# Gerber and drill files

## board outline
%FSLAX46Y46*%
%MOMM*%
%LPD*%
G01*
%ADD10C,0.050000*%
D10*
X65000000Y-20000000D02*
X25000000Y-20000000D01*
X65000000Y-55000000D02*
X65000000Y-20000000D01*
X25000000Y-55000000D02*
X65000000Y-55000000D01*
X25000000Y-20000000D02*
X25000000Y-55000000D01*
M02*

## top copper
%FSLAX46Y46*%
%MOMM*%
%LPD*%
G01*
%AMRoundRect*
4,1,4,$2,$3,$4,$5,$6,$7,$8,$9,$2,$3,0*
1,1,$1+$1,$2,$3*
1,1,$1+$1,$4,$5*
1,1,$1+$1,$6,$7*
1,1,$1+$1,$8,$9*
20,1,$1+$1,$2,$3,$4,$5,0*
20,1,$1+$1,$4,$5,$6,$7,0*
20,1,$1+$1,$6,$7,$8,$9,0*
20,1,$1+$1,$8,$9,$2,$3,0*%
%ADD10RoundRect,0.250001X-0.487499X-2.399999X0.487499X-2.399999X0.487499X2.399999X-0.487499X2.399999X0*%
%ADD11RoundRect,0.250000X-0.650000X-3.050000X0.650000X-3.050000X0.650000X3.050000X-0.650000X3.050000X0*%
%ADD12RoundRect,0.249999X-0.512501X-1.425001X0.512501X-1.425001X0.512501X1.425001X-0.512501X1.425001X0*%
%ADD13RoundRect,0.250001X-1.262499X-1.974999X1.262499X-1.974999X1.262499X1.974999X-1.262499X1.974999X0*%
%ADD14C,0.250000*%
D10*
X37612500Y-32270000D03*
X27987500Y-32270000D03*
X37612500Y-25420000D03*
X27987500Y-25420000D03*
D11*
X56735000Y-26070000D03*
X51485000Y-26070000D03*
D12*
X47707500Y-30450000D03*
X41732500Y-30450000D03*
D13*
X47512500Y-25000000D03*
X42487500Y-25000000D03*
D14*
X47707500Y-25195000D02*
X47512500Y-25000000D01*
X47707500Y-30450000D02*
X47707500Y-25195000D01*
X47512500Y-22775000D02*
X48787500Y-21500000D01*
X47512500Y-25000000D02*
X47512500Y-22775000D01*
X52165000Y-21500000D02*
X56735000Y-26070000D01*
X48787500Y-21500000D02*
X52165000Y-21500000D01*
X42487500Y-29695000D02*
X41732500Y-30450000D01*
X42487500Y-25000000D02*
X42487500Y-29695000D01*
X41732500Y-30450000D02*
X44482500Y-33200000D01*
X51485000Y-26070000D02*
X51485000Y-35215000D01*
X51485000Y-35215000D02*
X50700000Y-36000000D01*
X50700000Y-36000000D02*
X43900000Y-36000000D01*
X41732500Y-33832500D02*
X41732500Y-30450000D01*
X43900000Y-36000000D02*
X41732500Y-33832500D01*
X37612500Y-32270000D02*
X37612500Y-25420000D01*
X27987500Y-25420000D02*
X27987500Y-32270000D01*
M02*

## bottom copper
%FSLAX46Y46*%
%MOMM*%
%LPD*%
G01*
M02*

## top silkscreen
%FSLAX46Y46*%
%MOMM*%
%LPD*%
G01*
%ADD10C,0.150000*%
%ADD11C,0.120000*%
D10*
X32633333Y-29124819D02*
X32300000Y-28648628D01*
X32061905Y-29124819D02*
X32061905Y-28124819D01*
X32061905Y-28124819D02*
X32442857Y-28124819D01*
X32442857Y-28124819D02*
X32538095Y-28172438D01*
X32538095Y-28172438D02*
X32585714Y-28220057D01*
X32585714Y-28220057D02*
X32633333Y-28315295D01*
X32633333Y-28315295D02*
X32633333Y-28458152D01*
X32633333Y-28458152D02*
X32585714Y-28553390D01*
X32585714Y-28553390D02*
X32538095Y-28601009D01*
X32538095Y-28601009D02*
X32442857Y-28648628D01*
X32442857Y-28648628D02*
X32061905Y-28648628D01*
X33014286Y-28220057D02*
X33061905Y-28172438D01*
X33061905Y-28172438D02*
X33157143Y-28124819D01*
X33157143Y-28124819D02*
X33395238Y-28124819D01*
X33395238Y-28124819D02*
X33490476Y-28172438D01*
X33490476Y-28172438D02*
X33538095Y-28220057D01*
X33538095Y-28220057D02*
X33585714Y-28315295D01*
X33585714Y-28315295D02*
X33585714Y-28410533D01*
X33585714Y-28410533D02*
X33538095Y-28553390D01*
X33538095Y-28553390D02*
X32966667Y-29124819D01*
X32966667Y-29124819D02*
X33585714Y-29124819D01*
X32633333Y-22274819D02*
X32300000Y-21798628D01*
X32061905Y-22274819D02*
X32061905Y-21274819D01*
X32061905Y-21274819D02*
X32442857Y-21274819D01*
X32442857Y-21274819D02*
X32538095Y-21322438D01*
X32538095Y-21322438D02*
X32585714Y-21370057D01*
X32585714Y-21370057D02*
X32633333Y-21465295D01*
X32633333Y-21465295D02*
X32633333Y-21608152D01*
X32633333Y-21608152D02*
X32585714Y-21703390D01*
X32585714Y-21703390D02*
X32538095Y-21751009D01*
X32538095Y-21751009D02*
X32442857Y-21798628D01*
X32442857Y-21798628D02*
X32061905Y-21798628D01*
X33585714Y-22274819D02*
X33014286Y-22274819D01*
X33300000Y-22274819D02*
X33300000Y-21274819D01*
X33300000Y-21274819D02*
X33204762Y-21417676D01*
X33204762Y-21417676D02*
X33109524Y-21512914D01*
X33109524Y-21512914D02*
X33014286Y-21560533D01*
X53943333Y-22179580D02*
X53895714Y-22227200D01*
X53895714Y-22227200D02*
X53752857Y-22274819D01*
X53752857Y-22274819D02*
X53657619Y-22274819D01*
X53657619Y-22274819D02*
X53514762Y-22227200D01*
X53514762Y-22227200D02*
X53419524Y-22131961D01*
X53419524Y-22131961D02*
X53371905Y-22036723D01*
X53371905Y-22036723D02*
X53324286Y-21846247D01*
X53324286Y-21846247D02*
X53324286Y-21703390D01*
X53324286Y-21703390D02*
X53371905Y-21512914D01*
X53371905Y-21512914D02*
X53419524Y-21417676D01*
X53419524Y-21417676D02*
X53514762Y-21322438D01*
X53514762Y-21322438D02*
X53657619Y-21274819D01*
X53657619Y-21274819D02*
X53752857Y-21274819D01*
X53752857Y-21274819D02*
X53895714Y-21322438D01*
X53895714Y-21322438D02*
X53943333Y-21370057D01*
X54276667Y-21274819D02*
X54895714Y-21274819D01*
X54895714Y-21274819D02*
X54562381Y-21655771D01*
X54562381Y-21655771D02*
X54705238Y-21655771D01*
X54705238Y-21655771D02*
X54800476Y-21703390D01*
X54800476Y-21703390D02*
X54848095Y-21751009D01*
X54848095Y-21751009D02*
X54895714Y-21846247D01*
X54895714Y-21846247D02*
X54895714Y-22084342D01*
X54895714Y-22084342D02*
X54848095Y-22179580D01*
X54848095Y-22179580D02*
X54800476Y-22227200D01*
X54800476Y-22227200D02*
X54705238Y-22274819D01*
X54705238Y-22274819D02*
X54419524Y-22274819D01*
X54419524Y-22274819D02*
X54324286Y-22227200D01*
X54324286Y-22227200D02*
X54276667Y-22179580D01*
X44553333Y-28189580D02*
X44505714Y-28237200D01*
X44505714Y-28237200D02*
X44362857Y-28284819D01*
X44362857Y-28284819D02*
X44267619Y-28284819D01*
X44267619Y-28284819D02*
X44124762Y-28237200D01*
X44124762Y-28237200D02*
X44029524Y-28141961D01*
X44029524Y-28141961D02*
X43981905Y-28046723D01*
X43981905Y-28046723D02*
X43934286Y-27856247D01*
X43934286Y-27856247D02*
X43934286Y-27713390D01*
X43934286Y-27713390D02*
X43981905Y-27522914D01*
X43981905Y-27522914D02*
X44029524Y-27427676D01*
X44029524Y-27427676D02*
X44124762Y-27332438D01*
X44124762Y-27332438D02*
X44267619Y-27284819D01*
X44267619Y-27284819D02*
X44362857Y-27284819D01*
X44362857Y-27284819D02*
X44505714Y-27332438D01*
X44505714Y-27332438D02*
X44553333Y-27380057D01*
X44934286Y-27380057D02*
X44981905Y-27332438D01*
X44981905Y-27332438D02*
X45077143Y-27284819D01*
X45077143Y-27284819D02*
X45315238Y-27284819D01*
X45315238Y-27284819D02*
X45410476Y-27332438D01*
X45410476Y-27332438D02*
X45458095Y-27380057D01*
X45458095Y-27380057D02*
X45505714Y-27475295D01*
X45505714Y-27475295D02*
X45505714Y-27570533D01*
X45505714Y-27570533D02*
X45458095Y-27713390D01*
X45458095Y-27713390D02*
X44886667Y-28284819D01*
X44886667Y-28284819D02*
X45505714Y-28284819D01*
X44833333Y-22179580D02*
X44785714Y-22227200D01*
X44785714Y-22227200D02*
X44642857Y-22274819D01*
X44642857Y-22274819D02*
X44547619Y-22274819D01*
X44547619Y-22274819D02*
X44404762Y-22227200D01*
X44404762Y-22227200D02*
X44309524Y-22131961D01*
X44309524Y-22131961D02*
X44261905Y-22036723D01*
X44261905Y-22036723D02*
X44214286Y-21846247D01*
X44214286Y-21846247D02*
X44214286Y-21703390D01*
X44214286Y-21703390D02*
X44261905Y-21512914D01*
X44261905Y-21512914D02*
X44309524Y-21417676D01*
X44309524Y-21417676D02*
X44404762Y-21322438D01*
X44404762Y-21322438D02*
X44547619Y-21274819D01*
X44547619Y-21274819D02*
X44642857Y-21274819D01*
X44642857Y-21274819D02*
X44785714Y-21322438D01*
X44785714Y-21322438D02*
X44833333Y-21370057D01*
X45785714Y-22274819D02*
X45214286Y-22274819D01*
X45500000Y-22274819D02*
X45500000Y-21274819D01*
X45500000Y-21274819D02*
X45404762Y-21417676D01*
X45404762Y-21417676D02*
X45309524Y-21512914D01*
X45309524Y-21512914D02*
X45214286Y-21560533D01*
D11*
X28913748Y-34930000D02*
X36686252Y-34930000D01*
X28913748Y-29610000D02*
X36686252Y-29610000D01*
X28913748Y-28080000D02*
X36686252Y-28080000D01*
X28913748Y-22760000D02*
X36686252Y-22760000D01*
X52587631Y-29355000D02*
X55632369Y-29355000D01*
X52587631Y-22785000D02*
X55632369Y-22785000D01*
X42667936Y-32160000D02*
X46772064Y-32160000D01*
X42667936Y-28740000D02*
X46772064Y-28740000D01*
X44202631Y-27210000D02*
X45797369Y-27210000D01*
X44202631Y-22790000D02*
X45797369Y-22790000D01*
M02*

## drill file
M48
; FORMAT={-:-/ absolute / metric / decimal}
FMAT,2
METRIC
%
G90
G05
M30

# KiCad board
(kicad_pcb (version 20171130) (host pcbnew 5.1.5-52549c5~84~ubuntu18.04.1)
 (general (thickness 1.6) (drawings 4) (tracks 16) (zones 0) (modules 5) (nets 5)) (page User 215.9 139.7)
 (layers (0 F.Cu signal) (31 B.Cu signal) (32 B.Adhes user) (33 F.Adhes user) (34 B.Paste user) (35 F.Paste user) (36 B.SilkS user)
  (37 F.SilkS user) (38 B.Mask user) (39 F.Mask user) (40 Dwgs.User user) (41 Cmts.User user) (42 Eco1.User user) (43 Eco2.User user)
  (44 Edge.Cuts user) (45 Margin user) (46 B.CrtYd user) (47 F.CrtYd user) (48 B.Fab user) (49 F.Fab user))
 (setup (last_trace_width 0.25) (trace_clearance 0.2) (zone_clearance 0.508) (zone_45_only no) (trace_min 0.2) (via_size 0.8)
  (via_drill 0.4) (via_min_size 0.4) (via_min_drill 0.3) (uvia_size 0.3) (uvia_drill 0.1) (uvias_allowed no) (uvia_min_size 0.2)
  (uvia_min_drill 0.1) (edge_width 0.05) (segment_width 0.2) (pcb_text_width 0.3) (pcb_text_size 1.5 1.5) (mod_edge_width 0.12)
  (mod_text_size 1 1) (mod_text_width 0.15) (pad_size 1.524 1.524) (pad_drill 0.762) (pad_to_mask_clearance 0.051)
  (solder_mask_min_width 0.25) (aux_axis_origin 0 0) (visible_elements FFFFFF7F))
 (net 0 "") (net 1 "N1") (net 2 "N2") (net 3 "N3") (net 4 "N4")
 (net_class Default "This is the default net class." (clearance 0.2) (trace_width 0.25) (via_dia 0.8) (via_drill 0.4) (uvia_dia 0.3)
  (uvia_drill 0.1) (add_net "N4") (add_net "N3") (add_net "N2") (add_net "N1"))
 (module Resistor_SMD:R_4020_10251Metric (layer F.Cu) (at 32.8 32.27)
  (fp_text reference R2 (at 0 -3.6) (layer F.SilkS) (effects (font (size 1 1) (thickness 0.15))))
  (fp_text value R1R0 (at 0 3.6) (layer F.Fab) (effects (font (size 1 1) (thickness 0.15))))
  (fp_line (start -3.886252 2.66) (end 3.886252 2.66) (layer F.SilkS) (width 0.12))
  (fp_line (start -3.886252 -2.66) (end 3.886252 -2.66) (layer F.SilkS) (width 0.12))
  (pad 2 smd roundrect (at 4.8125 0) (size 1.475 5.3) (layers F.Cu F.Paste F.Mask) (roundrect_rratio 0.169492) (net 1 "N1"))
  (pad 1 smd roundrect (at -4.8125 0) (size 1.475 5.3) (layers F.Cu F.Paste F.Mask) (roundrect_rratio 0.169492) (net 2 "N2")))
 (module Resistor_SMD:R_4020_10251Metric (layer F.Cu) (at 32.8 25.42)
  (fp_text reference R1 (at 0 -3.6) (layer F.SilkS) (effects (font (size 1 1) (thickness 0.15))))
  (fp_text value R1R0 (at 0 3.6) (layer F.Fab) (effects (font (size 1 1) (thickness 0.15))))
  (fp_line (start -3.886252 2.66) (end 3.886252 2.66) (layer F.SilkS) (width 0.12))
  (fp_line (start -3.886252 -2.66) (end 3.886252 -2.66) (layer F.SilkS) (width 0.12))
  (pad 2 smd roundrect (at 4.8125 0) (size 1.475 5.3) (layers F.Cu F.Paste F.Mask) (roundrect_rratio 0.169492) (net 1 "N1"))
  (pad 1 smd roundrect (at -4.8125 0) (size 1.475 5.3) (layers F.Cu F.Paste F.Mask) (roundrect_rratio 0.169492) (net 2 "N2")))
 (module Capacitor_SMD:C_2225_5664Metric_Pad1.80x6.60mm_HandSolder (layer F.Cu) (at 54.11 26.07)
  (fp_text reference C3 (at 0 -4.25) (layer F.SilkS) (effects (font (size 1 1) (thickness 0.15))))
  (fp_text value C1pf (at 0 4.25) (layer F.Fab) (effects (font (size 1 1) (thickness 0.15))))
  (fp_line (start -1.522369 3.285) (end 1.522369 3.285) (layer F.SilkS) (width 0.12))
  (fp_line (start -1.522369 -3.285) (end 1.522369 -3.285) (layer F.SilkS) (width 0.12))
  (pad 2 smd roundrect (at 2.625 0) (size 1.8 6.6) (layers F.Cu F.Paste F.Mask) (roundrect_rratio 0.138889) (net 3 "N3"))
  (pad 1 smd roundrect (at -2.625 0) (size 1.8 6.6) (layers F.Cu F.Paste F.Mask) (roundrect_rratio 0.138889) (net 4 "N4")))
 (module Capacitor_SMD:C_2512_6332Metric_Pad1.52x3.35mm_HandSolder (layer F.Cu) (at 44.72 30.45)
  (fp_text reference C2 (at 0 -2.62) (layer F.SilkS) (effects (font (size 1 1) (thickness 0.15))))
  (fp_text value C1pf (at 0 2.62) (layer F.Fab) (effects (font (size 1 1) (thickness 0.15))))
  (fp_line (start -2.052064 1.71) (end 2.052064 1.71) (layer F.SilkS) (width 0.12))
  (fp_line (start -2.052064 -1.71) (end 2.052064 -1.71) (layer F.SilkS) (width 0.12))
  (pad 2 smd roundrect (at 2.9875 0) (size 1.525 3.35) (layers F.Cu F.Paste F.Mask) (roundrect_rratio 0.163934) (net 3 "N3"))
  (pad 1 smd roundrect (at -2.9875 0) (size 1.525 3.35) (layers F.Cu F.Paste F.Mask) (roundrect_rratio 0.163934) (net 4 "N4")))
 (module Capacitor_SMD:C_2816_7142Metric (layer F.Cu) (at 45 25)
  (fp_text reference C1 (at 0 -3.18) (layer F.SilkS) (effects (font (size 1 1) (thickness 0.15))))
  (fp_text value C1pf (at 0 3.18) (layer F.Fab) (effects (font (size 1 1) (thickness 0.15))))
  (fp_line (start -0.797369 2.21) (end 0.797369 2.21) (layer F.SilkS) (width 0.12))
  (fp_line (start -0.797369 -2.21) (end 0.797369 -2.21) (layer F.SilkS) (width 0.12))
  (pad 2 smd roundrect (at 2.5125 0) (size 3.025 4.45) (layers F.Cu F.Paste F.Mask) (roundrect_rratio 0.082645) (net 3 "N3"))
  (pad 1 smd roundrect (at -2.5125 0) (size 3.025 4.45) (layers F.Cu F.Paste F.Mask) (roundrect_rratio 0.082645) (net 4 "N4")))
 (gr_line (start 65 20) (end 25 20) (layer Edge.Cuts) (width 0.05))
 (gr_line (start 65 55) (end 65 20) (layer Edge.Cuts) (width 0.05))
 (gr_line (start 25 55) (end 65 55) (layer Edge.Cuts) (width 0.05))
 (gr_line (start 25 20) (end 25 55) (layer Edge.Cuts) (width 0.05))
 (segment (start 47.7075 25.195) (end 47.5125 25) (width 0.25) (layer F.Cu) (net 3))
 (segment (start 47.7075 30.45) (end 47.7075 25.195) (width 0.25) (layer F.Cu) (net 3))
 (segment (start 47.5125 22.775) (end 48.7875 21.5) (width 0.25) (layer F.Cu) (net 3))
 (segment (start 47.5125 25) (end 47.5125 22.775) (width 0.25) (layer F.Cu) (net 3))
 (segment (start 52.165 21.5) (end 56.735 26.07) (width 0.25) (layer F.Cu) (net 3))
 (segment (start 48.7875 21.5) (end 52.165 21.5) (width 0.25) (layer F.Cu) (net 3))
 (segment (start 42.4875 29.695) (end 41.7325 30.45) (width 0.25) (layer F.Cu) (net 4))
 (segment (start 42.4875 25) (end 42.4875 29.695) (width 0.25) (layer F.Cu) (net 4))
 (segment (start 41.7325 30.45) (end 44.4825 33.2) (width 0.25) (layer F.Cu) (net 4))
 (segment (start 51.485 26.07) (end 51.485 35.215) (width 0.25) (layer F.Cu) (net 4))
 (segment (start 51.485 35.215) (end 50.7 36) (width 0.25) (layer F.Cu) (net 4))
 (segment (start 50.7 36) (end 43.9 36) (width 0.25) (layer F.Cu) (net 4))
 (segment (start 41.7325 33.8325) (end 41.7325 30.45) (width 0.25) (layer F.Cu) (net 4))
 (segment (start 43.9 36) (end 41.7325 33.8325) (width 0.25) (layer F.Cu) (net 4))
 (segment (start 37.6125 32.27) (end 37.6125 25.42) (width 0.25) (layer F.Cu) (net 1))
 (segment (start 27.9875 25.42) (end 27.9875 32.27) (width 0.25) (layer F.Cu) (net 2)))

